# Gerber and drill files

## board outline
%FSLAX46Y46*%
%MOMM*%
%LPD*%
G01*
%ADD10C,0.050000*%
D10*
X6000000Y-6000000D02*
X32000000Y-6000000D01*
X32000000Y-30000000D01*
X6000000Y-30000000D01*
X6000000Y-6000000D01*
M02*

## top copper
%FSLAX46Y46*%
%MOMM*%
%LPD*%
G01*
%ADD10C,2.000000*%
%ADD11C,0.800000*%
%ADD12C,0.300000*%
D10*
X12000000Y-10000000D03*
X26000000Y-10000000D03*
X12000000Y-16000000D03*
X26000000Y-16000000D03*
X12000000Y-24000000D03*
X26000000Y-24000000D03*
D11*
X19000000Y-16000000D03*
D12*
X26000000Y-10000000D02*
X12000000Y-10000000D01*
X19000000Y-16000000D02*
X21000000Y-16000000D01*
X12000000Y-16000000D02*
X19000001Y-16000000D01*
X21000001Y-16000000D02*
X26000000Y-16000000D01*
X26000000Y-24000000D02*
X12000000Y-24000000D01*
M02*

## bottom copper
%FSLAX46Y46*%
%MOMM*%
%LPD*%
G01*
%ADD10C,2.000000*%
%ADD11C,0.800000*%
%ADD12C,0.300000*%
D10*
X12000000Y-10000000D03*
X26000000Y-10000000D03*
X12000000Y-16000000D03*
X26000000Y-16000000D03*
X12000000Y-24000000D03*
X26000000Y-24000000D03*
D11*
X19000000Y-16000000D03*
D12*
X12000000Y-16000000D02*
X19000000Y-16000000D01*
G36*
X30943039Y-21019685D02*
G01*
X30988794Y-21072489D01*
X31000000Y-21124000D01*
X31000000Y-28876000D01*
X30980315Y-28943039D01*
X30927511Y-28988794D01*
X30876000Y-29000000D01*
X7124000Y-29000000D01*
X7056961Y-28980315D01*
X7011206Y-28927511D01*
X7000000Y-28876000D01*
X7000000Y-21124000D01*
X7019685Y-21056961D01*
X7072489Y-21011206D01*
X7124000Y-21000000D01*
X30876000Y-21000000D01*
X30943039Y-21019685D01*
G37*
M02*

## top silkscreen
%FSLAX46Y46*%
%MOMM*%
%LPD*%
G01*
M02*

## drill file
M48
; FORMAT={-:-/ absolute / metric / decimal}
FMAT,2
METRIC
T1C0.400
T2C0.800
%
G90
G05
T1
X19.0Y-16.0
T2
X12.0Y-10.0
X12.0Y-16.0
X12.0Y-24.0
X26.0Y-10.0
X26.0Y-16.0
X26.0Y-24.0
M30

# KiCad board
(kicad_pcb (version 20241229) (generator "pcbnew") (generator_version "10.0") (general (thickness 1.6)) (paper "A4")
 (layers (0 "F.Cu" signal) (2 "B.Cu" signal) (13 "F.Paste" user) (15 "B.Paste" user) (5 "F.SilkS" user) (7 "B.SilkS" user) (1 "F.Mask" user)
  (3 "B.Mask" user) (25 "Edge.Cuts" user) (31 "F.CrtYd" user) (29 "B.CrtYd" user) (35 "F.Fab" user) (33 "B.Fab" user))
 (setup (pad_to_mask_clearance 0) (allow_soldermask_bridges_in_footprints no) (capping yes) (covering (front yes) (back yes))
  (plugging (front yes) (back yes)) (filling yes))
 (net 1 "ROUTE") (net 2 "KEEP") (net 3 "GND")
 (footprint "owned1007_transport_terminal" (layer "F.Cu") (at 12 10)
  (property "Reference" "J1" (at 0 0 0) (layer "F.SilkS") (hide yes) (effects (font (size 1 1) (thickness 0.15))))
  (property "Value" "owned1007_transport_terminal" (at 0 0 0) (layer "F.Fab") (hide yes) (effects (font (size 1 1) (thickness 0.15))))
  (pad "1" thru_hole circle (at 0 0) (size 2 2) (drill 0.8) (layers "*.Cu" "*.Mask") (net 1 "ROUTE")))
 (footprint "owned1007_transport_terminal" (layer "F.Cu") (at 26 10)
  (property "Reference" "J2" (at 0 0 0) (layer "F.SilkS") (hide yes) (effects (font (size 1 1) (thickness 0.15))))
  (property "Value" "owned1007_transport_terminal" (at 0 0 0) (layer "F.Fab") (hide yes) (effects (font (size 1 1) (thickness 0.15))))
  (pad "1" thru_hole circle (at 0 0) (size 2 2) (drill 0.8) (layers "*.Cu" "*.Mask") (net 1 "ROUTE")))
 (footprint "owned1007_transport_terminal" (layer "F.Cu") (at 12 16)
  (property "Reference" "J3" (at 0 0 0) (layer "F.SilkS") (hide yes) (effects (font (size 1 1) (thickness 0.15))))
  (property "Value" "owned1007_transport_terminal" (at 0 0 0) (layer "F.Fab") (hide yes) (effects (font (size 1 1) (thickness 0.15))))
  (pad "1" thru_hole circle (at 0 0) (size 2 2) (drill 0.8) (layers "*.Cu" "*.Mask") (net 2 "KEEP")))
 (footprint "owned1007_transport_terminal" (layer "F.Cu") (at 26 16)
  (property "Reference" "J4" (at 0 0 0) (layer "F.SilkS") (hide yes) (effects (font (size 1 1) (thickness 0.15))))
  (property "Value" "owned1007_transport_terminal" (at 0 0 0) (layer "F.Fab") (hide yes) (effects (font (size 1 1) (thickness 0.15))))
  (pad "1" thru_hole circle (at 0 0) (size 2 2) (drill 0.8) (layers "*.Cu" "*.Mask") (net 2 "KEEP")))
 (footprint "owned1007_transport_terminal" (layer "F.Cu") (at 12 24)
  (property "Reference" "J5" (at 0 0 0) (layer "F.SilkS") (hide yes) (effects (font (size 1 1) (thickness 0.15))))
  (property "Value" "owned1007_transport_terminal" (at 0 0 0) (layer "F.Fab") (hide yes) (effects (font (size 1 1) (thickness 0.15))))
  (pad "1" thru_hole circle (at 0 0) (size 2 2) (drill 0.8) (layers "*.Cu" "*.Mask") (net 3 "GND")))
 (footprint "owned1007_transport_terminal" (layer "F.Cu") (at 26 24)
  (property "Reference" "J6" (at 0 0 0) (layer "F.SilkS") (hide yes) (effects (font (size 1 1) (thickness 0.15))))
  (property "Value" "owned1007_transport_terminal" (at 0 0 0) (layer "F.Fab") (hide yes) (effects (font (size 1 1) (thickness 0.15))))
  (pad "1" thru_hole circle (at 0 0) (size 2 2) (drill 0.8) (layers "*.Cu" "*.Mask") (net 3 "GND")))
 (gr_rect (start 6 6) (end 32 30) (stroke (width 0.05) (type default)) (fill none) (layer "Edge.Cuts"))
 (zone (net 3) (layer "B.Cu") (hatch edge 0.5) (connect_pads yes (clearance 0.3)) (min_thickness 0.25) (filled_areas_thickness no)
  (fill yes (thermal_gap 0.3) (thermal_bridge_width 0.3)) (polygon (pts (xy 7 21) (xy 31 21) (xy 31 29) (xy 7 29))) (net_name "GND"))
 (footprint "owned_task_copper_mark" (layer "F.Cu") (at 10 28)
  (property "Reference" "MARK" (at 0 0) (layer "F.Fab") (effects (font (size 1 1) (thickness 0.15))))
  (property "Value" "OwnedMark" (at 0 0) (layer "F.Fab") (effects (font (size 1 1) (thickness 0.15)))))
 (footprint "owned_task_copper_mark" (layer "F.Cu") (at 13 28)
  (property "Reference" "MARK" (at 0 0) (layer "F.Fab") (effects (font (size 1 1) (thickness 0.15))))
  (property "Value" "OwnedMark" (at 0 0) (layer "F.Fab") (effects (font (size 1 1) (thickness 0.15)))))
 (segment (start 26 10) (end 12 10) (width 0.3) (layer "F.Cu") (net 1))
 (segment (start 19 16) (end 21 16) (width 0.3) (layer "F.Cu") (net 2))
 (segment (start 12 16) (end 19.000001 16) (width 0.3) (layer "F.Cu") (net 2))
 (segment (start 21.000001 16) (end 26 16) (width 0.3) (layer "F.Cu") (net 2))
 (via (at 19 16) (size 0.8) (drill 0.4) (layers "F.Cu" "B.Cu") (free yes) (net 2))
 (segment (start 12 16) (end 19 16) (width 0.3) (layer "B.Cu") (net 2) (locked yes))
 (segment (start 26 24) (end 12 24) (width 0.3) (layer "F.Cu") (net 3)))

